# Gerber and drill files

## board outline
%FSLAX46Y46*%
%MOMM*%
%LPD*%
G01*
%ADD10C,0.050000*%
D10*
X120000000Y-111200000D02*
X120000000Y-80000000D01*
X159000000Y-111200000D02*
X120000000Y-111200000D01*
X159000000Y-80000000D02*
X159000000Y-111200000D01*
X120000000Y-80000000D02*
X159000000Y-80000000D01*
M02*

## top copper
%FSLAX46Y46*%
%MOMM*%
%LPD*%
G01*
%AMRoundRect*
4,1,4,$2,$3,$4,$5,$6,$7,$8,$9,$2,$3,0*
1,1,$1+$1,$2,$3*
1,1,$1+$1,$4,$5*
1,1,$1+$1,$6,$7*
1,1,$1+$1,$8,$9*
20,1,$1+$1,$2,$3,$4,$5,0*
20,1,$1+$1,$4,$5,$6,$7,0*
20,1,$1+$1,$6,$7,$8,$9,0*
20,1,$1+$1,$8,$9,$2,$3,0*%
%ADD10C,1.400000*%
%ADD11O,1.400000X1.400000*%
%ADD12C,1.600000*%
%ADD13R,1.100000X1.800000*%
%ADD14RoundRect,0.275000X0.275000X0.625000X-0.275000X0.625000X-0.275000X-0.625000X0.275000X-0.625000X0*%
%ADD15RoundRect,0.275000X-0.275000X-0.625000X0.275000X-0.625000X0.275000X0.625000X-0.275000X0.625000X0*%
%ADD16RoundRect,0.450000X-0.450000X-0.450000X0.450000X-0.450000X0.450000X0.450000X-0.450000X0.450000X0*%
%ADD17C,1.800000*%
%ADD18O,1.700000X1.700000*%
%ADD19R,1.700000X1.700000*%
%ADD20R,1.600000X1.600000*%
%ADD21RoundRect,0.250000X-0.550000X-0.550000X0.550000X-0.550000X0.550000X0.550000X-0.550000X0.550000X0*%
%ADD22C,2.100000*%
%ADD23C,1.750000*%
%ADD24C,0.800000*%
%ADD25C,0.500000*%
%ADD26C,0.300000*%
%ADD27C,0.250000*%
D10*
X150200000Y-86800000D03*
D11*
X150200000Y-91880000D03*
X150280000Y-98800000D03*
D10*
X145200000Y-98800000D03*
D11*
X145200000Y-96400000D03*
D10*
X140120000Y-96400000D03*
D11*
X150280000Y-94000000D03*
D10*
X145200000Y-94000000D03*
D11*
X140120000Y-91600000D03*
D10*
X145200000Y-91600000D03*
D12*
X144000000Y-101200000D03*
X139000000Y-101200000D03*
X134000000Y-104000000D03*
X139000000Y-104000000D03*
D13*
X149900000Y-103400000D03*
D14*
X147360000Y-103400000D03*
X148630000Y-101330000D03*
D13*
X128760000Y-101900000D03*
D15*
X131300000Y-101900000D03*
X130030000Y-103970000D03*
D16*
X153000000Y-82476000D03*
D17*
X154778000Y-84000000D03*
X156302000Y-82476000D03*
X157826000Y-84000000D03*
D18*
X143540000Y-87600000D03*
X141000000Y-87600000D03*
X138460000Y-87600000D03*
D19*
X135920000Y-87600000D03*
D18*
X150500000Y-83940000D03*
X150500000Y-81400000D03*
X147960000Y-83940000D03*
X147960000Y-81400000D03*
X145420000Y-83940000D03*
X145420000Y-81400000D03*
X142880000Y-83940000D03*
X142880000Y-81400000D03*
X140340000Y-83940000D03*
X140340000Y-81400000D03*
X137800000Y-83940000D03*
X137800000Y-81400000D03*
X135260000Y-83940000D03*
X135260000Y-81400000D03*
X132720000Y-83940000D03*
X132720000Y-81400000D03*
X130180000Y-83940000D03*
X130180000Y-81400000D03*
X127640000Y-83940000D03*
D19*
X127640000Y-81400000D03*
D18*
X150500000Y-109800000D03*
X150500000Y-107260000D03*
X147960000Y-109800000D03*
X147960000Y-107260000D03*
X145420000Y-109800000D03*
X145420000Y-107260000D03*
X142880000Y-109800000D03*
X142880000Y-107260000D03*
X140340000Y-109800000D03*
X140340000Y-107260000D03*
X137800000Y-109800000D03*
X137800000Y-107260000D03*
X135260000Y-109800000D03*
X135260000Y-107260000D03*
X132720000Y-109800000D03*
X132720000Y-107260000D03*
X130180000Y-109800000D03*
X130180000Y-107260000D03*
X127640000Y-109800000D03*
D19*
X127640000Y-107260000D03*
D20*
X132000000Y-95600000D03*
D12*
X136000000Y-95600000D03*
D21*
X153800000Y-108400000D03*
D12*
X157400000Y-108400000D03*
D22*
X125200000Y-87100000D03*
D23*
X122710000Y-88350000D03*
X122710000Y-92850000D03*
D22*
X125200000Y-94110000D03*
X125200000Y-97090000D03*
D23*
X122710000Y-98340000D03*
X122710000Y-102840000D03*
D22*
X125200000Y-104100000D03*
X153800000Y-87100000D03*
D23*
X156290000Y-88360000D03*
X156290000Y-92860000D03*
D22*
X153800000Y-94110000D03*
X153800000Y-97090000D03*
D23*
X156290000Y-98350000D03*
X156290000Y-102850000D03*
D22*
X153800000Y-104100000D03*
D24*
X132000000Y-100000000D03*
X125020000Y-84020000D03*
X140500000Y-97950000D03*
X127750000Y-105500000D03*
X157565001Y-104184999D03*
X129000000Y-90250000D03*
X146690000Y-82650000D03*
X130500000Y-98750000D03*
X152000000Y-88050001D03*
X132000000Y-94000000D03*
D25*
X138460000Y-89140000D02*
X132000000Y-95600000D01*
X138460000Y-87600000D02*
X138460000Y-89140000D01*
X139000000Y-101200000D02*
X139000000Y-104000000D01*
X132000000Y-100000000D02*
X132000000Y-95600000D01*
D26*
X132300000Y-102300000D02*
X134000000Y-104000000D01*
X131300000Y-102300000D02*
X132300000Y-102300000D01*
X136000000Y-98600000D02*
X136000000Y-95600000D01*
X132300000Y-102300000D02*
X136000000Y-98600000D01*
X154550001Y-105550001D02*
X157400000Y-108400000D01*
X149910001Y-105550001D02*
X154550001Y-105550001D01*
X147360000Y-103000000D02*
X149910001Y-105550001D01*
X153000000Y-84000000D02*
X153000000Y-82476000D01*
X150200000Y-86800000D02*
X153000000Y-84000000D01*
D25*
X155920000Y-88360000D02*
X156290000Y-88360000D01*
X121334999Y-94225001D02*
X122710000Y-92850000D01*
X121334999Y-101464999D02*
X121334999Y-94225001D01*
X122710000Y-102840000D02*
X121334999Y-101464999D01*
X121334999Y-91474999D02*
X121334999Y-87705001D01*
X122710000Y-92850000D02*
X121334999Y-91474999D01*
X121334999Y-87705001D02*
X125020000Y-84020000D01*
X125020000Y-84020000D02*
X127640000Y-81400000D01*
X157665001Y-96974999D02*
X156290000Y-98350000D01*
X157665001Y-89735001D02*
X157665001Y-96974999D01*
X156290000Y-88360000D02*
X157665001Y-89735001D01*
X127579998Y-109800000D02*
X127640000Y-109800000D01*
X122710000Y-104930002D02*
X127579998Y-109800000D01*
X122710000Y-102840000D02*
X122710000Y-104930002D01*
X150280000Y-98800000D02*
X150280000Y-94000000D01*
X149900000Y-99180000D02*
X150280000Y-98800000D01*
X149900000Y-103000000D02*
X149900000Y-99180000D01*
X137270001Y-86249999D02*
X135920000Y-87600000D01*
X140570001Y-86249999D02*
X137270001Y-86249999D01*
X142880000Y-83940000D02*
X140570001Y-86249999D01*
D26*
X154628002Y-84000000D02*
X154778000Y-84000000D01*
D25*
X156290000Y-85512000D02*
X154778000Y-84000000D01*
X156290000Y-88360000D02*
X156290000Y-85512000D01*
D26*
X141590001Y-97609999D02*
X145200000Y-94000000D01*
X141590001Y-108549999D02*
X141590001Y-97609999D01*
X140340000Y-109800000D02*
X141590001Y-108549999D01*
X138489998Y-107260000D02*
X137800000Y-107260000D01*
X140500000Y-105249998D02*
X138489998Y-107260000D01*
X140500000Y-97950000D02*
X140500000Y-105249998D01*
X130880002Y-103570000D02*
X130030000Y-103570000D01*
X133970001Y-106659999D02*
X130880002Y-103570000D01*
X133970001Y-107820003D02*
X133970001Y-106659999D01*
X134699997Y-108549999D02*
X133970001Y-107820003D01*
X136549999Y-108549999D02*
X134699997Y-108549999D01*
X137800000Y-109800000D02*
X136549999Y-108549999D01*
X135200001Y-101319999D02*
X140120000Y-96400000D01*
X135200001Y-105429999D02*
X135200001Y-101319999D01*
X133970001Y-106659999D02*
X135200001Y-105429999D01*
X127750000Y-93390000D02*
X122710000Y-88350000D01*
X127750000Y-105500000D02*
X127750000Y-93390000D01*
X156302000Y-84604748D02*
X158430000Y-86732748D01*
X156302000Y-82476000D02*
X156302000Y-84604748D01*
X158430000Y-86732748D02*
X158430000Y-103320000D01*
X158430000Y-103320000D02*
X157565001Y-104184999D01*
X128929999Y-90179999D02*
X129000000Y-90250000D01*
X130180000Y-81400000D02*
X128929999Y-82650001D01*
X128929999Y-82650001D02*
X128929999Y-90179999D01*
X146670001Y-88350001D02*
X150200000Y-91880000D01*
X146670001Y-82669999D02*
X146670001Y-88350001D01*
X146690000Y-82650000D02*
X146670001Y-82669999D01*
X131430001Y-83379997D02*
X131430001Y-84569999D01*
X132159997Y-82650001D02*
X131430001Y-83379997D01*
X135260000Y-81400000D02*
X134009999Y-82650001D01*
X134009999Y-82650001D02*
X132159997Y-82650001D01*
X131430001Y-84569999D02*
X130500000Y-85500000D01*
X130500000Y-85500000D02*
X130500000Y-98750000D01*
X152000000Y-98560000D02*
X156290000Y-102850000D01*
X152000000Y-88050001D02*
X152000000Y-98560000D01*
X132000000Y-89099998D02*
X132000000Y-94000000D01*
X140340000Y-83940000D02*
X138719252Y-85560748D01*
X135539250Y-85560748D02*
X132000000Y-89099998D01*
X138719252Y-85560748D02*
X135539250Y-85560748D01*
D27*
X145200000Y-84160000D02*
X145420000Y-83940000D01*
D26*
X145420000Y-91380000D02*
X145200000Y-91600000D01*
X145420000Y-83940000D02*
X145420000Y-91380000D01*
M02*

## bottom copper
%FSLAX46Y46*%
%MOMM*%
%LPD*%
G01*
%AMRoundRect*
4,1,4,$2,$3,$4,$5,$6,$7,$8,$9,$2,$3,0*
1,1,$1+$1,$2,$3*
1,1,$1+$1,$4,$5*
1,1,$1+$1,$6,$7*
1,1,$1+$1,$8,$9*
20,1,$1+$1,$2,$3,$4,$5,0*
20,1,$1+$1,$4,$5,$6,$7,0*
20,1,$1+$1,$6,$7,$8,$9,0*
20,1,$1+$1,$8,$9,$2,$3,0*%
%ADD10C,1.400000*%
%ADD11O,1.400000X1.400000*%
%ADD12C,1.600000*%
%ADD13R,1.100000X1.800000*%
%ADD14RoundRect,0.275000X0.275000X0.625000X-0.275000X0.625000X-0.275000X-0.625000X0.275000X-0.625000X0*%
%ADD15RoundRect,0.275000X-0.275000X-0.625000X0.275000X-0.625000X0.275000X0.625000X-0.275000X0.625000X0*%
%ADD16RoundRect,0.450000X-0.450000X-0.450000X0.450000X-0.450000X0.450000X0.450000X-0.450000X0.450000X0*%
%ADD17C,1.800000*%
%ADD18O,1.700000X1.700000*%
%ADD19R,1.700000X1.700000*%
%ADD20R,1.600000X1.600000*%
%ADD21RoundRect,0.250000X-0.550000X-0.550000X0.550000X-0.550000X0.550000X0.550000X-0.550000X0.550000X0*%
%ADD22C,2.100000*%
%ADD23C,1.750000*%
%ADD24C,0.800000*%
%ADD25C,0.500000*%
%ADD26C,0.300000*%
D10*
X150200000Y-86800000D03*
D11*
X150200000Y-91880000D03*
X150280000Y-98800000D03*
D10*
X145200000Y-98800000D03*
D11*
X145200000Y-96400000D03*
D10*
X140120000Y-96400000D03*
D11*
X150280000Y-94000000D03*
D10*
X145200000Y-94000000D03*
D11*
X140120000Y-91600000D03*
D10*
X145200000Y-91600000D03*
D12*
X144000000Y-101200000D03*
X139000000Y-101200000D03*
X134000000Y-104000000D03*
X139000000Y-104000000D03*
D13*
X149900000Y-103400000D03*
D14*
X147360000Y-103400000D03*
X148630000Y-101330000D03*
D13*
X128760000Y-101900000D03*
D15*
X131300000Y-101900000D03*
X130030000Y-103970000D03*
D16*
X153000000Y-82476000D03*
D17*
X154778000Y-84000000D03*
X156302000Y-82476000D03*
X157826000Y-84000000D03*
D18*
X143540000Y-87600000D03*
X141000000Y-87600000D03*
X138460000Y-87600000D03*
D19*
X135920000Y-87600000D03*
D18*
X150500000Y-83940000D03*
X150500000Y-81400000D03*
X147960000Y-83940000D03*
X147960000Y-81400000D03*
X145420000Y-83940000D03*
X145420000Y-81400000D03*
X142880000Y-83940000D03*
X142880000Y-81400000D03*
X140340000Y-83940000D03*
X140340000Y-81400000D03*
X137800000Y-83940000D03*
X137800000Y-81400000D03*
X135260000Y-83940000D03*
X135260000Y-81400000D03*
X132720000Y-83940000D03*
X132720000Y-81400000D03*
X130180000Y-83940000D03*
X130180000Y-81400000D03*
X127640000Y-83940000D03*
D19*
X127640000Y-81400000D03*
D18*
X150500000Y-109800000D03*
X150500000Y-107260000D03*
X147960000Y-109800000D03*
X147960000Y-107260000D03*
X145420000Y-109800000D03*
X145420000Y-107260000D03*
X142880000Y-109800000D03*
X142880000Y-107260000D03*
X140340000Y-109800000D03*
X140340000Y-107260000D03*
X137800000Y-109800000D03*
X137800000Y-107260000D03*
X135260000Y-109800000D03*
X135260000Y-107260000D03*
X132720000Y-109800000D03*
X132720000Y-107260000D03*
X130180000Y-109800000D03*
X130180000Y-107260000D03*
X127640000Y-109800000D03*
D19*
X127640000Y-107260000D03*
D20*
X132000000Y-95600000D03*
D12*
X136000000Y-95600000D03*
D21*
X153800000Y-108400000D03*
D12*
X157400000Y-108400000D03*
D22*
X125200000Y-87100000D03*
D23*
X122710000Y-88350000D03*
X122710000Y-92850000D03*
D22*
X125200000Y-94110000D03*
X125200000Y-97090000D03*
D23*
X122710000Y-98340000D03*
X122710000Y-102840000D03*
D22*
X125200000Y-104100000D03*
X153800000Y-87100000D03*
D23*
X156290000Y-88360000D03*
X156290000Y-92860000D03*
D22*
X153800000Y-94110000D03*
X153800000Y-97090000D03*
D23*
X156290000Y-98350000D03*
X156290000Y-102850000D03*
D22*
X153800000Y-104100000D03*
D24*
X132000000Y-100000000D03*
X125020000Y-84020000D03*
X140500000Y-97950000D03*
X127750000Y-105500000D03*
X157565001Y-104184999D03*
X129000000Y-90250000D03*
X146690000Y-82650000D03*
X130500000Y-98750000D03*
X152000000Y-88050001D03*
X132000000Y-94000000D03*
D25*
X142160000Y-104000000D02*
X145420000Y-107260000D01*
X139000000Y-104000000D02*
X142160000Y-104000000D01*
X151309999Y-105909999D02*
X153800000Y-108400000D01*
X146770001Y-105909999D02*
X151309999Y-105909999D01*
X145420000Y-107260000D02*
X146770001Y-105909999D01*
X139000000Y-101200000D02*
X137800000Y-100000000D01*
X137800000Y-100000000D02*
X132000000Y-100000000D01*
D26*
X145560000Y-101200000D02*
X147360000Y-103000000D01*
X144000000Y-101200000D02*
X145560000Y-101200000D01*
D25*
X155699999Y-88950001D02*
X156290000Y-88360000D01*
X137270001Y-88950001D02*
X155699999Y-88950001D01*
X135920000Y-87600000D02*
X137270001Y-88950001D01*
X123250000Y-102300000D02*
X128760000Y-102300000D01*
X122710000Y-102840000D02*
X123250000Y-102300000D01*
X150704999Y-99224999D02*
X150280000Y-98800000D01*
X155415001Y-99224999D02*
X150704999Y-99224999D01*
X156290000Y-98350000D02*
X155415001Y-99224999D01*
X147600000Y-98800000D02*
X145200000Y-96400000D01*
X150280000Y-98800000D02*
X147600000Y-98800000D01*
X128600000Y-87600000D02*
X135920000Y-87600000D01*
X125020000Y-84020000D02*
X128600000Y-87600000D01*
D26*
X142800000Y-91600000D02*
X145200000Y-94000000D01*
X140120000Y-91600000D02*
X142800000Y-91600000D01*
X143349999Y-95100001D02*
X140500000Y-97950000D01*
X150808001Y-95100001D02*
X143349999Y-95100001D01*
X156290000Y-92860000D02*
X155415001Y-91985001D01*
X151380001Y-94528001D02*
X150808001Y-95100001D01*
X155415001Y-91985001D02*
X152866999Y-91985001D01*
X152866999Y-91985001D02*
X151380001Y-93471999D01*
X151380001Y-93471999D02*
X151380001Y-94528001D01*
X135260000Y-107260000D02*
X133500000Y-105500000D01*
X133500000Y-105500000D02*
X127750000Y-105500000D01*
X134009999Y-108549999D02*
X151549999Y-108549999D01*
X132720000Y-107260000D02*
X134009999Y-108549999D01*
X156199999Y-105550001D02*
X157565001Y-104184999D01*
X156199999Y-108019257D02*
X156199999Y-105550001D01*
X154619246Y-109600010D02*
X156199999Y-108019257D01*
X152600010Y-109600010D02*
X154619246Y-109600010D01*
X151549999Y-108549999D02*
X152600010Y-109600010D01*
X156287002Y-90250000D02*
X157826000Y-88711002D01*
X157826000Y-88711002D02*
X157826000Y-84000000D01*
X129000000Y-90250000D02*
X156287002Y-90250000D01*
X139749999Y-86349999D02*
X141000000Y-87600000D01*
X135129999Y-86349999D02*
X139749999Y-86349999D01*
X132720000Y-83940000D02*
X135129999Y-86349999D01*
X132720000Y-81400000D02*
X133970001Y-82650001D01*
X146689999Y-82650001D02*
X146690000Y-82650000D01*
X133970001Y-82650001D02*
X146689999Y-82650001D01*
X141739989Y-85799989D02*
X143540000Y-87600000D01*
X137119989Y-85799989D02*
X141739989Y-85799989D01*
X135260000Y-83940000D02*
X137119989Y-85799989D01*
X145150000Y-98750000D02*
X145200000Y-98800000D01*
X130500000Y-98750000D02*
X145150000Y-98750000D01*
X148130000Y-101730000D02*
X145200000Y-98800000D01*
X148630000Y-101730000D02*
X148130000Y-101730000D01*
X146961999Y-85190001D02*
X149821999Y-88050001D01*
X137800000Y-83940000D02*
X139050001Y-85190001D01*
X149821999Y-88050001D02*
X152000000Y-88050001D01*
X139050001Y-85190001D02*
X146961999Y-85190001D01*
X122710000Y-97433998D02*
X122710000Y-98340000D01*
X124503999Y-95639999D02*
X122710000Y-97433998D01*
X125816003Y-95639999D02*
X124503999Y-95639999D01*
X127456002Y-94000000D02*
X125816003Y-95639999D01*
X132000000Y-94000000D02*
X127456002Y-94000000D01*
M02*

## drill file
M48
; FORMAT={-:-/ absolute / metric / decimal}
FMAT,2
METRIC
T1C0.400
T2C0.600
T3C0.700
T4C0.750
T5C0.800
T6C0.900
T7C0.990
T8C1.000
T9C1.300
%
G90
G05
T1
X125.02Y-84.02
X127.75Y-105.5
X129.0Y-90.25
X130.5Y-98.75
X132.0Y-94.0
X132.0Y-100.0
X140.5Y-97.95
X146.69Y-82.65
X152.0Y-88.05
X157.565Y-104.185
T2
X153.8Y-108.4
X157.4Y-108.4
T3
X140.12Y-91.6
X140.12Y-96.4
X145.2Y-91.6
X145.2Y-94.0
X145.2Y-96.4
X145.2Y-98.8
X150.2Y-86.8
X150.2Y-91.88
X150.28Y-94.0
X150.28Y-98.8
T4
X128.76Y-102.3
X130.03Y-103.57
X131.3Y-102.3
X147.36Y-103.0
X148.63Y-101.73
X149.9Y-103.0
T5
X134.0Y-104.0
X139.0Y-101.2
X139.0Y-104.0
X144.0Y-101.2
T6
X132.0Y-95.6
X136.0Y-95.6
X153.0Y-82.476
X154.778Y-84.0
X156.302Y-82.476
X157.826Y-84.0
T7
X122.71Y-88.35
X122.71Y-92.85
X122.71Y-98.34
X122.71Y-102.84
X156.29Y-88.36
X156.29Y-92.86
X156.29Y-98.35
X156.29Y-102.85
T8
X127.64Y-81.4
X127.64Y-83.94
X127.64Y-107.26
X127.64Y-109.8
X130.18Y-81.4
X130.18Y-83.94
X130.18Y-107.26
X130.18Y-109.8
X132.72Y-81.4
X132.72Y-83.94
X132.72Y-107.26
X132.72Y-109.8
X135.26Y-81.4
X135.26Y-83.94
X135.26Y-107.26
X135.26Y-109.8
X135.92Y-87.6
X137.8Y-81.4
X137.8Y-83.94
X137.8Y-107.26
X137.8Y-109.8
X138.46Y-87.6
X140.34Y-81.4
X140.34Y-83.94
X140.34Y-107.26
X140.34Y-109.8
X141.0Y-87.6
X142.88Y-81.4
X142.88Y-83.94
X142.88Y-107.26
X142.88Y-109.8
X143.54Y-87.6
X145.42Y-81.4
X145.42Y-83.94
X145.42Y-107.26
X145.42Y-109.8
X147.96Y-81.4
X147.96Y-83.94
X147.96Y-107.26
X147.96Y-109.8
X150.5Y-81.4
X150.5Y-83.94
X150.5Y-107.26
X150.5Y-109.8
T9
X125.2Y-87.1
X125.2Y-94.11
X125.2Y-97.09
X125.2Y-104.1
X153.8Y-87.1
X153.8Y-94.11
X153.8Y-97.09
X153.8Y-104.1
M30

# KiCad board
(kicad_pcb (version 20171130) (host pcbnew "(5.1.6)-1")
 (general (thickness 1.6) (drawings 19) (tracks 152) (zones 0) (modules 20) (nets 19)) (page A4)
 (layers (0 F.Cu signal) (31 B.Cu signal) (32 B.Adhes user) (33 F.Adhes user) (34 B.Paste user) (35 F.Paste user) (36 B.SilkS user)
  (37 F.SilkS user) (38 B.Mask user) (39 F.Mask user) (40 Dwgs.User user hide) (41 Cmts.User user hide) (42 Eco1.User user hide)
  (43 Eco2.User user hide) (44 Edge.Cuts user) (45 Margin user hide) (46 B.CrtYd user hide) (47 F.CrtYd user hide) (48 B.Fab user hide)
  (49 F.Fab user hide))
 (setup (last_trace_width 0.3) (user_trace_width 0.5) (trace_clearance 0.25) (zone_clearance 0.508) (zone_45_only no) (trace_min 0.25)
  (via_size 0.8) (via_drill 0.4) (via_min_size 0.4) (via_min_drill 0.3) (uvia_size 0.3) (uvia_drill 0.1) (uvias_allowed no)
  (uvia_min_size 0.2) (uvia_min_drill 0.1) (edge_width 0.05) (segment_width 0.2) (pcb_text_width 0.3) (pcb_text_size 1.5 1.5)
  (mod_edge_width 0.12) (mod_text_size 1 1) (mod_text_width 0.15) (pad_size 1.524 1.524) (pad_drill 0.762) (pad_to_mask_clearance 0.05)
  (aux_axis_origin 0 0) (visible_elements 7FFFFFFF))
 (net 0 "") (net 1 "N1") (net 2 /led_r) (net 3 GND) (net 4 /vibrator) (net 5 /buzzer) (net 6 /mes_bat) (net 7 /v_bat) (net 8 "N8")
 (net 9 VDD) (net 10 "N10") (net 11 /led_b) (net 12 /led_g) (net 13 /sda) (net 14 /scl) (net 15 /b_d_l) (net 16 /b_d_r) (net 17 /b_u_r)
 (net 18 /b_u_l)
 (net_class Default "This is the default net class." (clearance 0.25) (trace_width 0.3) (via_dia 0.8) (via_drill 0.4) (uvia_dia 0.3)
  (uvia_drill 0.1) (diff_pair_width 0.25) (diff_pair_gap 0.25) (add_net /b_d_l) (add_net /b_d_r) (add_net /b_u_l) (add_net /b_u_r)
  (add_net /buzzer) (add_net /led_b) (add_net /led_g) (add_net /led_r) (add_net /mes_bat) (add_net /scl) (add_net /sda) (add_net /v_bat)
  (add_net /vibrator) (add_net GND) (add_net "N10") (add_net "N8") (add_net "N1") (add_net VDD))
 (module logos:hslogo (layer F.Cu) (at 122.7 108)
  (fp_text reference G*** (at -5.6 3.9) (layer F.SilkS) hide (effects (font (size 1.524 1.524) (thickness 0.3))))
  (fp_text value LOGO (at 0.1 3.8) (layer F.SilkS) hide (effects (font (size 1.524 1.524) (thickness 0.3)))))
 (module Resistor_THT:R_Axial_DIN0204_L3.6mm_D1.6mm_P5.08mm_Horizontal (layer B.Cu) (at 150.2 86.8 270)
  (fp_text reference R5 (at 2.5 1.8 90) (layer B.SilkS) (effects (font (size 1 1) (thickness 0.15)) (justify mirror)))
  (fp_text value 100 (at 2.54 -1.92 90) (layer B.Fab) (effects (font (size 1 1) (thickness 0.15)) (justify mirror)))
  (pad 1 thru_hole circle (at 0 0 270) (size 1.4 1.4) (drill 0.7) (layers *.Cu *.Mask) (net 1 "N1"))
  (pad 2 thru_hole oval (at 5.08 0 270) (size 1.4 1.4) (drill 0.7) (layers *.Cu *.Mask) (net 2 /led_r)))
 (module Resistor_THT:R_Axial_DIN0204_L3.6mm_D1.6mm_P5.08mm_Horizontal (layer B.Cu) (at 145.2 98.8)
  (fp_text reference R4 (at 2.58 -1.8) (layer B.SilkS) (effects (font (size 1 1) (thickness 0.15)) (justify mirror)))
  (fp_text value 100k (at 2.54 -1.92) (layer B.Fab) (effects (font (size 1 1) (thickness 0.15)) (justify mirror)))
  (pad 2 thru_hole oval (at 5.08 0) (size 1.4 1.4) (drill 0.7) (layers *.Cu *.Mask) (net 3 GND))
  (pad 1 thru_hole circle (at 0 0) (size 1.4 1.4) (drill 0.7) (layers *.Cu *.Mask) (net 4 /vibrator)))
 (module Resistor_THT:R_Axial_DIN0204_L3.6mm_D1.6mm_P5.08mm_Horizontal (layer B.Cu) (at 140.12 96.4)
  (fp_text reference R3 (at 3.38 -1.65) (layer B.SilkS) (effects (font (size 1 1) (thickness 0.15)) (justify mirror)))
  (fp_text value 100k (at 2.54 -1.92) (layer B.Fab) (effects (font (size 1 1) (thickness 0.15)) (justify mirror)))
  (pad 2 thru_hole oval (at 5.08 0) (size 1.4 1.4) (drill 0.7) (layers *.Cu *.Mask) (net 3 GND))
  (pad 1 thru_hole circle (at 0 0) (size 1.4 1.4) (drill 0.7) (layers *.Cu *.Mask) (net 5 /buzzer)))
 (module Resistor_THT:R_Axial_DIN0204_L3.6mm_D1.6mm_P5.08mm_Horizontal (layer B.Cu) (at 145.2 94)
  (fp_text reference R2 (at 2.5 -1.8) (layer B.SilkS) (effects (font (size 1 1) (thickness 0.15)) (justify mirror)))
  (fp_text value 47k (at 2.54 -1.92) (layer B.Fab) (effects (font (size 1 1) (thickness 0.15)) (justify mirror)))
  (pad 2 thru_hole oval (at 5.08 0) (size 1.4 1.4) (drill 0.7) (layers *.Cu *.Mask) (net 3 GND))
  (pad 1 thru_hole circle (at 0 0) (size 1.4 1.4) (drill 0.7) (layers *.Cu *.Mask) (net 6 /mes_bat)))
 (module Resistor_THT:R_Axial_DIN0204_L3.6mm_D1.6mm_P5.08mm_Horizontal (layer B.Cu) (at 145.2 91.6 180)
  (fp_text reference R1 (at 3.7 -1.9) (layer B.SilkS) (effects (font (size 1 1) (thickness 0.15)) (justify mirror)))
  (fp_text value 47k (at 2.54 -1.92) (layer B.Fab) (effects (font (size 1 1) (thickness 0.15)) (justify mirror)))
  (pad 2 thru_hole oval (at 5.08 0 180) (size 1.4 1.4) (drill 0.7) (layers *.Cu *.Mask) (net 6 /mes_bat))
  (pad 1 thru_hole circle (at 0 0 180) (size 1.4 1.4) (drill 0.7) (layers *.Cu *.Mask) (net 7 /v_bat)))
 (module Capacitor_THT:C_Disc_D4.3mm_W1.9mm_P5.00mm (layer B.Cu) (at 139 101.2)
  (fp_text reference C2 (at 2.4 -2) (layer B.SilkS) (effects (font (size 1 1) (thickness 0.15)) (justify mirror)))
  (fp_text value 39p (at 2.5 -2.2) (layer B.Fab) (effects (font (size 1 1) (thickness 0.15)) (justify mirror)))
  (pad 2 thru_hole circle (at 5 0) (size 1.6 1.6) (drill 0.8) (layers *.Cu *.Mask) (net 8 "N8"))
  (pad 1 thru_hole circle (at 0 0) (size 1.6 1.6) (drill 0.8) (layers *.Cu *.Mask) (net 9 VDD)))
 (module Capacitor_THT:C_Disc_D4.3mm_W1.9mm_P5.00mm (layer B.Cu) (at 139 104 180)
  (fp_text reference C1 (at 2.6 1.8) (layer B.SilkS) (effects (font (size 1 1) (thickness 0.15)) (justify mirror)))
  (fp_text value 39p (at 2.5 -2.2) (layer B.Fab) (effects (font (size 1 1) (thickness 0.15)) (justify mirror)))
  (pad 2 thru_hole circle (at 5 0 180) (size 1.6 1.6) (drill 0.8) (layers *.Cu *.Mask) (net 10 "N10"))
  (pad 1 thru_hole circle (at 0 0 180) (size 1.6 1.6) (drill 0.8) (layers *.Cu *.Mask) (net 9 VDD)))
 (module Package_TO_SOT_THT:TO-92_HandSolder (layer B.Cu) (at 149.9 103 180)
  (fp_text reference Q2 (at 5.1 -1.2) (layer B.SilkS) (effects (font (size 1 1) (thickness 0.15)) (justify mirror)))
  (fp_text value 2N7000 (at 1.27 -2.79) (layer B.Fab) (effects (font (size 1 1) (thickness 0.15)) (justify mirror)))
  (pad 1 thru_hole rect (at 0 0 180) (size 1.1 1.8) (drill 0.75 (offset 0 -0.4)) (layers *.Cu *.Mask) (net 3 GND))
  (pad 3 thru_hole roundrect (at 2.54 0 180) (size 1.1 1.8) (drill 0.75 (offset 0 -0.4)) (layers *.Cu *.Mask) (roundrect_rratio 0.25)
   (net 8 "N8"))
  (pad 2 thru_hole roundrect (at 1.27 1.27 180) (size 1.1 1.8) (drill 0.75 (offset 0 0.4)) (layers *.Cu *.Mask) (roundrect_rratio 0.25)
   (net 4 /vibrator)))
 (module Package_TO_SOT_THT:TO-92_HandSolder (layer B.Cu) (at 128.76 102.3)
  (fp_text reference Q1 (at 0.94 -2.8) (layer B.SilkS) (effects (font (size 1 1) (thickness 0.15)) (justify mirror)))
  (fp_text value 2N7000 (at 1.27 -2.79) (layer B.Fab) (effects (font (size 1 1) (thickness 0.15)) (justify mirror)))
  (pad 1 thru_hole rect (at 0 0) (size 1.1 1.8) (drill 0.75 (offset 0 -0.4)) (layers *.Cu *.Mask) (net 3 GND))
  (pad 3 thru_hole roundrect (at 2.54 0) (size 1.1 1.8) (drill 0.75 (offset 0 -0.4)) (layers *.Cu *.Mask) (roundrect_rratio 0.25)
   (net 10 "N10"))
  (pad 2 thru_hole roundrect (at 1.27 1.27) (size 1.1 1.8) (drill 0.75 (offset 0 0.4)) (layers *.Cu *.Mask) (roundrect_rratio 0.25)
   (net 5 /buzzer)))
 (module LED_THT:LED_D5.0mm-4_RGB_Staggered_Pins (layer F.Cu) (at 153 82.476)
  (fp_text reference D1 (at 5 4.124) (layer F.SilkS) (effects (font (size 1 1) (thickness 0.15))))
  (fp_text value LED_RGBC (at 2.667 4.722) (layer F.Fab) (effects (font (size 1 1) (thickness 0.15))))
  (pad 1 thru_hole roundrect (at 0 0) (size 1.8 1.8) (drill 0.9) (layers *.Cu *.Mask) (roundrect_rratio 0.25) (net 1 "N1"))
  (pad 2 thru_hole circle (at 1.778 1.524) (size 1.8 1.8) (drill 0.9) (layers *.Cu *.Mask) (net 3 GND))
  (pad 3 thru_hole circle (at 3.302 0) (size 1.8 1.8) (drill 0.9) (layers *.Cu *.Mask) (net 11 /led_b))
  (pad 4 thru_hole circle (at 4.826 1.524) (size 1.8 1.8) (drill 0.9) (layers *.Cu *.Mask) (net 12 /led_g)))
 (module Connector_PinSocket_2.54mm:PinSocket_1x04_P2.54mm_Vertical (layer F.Cu) (at 135.92 87.6 90)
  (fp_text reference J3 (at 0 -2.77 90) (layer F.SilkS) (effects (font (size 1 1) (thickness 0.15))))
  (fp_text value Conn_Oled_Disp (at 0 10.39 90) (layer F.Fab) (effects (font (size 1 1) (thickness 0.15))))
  (pad 4 thru_hole oval (at 0 7.62 90) (size 1.7 1.7) (drill 1) (layers *.Cu *.Mask) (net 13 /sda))
  (pad 3 thru_hole oval (at 0 5.08 90) (size 1.7 1.7) (drill 1) (layers *.Cu *.Mask) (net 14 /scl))
  (pad 2 thru_hole oval (at 0 2.54 90) (size 1.7 1.7) (drill 1) (layers *.Cu *.Mask) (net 9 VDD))
  (pad 1 thru_hole rect (at 0 0 90) (size 1.7 1.7) (drill 1) (layers *.Cu *.Mask) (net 3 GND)))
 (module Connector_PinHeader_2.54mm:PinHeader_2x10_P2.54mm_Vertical (layer B.Cu) (at 127.64 81.4 270)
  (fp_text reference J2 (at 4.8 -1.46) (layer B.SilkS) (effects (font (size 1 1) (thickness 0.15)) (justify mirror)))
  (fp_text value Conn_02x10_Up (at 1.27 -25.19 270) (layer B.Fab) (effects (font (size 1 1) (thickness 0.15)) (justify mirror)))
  (pad 20 thru_hole oval (at 2.54 -22.86 270) (size 1.7 1.7) (drill 1) (layers *.Cu *.Mask))
  (pad 19 thru_hole oval (at 0 -22.86 270) (size 1.7 1.7) (drill 1) (layers *.Cu *.Mask))
  (pad 18 thru_hole oval (at 2.54 -20.32 270) (size 1.7 1.7) (drill 1) (layers *.Cu *.Mask))
  (pad 17 thru_hole oval (at 0 -20.32 270) (size 1.7 1.7) (drill 1) (layers *.Cu *.Mask))
  (pad 16 thru_hole oval (at 2.54 -17.78 270) (size 1.7 1.7) (drill 1) (layers *.Cu *.Mask) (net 7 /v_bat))
  (pad 15 thru_hole oval (at 0 -17.78 270) (size 1.7 1.7) (drill 1) (layers *.Cu *.Mask))
  (pad 14 thru_hole oval (at 2.54 -15.24 270) (size 1.7 1.7) (drill 1) (layers *.Cu *.Mask) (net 3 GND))
  (pad 13 thru_hole oval (at 0 -15.24 270) (size 1.7 1.7) (drill 1) (layers *.Cu *.Mask))
  (pad 12 thru_hole oval (at 2.54 -12.7 270) (size 1.7 1.7) (drill 1) (layers *.Cu *.Mask) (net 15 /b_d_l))
  (pad 11 thru_hole oval (at 0 -12.7 270) (size 1.7 1.7) (drill 1) (layers *.Cu *.Mask))
  (pad 10 thru_hole oval (at 2.54 -10.16 270) (size 1.7 1.7) (drill 1) (layers *.Cu *.Mask) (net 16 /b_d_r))
  (pad 9 thru_hole oval (at 0 -10.16 270) (size 1.7 1.7) (drill 1) (layers *.Cu *.Mask))
  (pad 8 thru_hole oval (at 2.54 -7.62 270) (size 1.7 1.7) (drill 1) (layers *.Cu *.Mask) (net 13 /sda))
  (pad 7 thru_hole oval (at 0 -7.62 270) (size 1.7 1.7) (drill 1) (layers *.Cu *.Mask) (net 4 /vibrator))
  (pad 6 thru_hole oval (at 2.54 -5.08 270) (size 1.7 1.7) (drill 1) (layers *.Cu *.Mask) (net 14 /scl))
  (pad 5 thru_hole oval (at 0 -5.08 270) (size 1.7 1.7) (drill 1) (layers *.Cu *.Mask) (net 2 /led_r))
  (pad 4 thru_hole oval (at 2.54 -2.54 270) (size 1.7 1.7) (drill 1) (layers *.Cu *.Mask))
  (pad 3 thru_hole oval (at 0 -2.54 270) (size 1.7 1.7) (drill 1) (layers *.Cu *.Mask) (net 12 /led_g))
  (pad 2 thru_hole oval (at 2.54 0 270) (size 1.7 1.7) (drill 1) (layers *.Cu *.Mask))
  (pad 1 thru_hole rect (at 0 0 270) (size 1.7 1.7) (drill 1) (layers *.Cu *.Mask) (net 3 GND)))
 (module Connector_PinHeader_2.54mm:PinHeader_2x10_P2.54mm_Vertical (layer B.Cu) (at 127.64 107.26 270)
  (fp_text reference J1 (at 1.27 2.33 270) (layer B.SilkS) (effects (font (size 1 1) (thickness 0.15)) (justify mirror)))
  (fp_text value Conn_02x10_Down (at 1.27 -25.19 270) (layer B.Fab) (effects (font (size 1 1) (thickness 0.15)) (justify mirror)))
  (pad 20 thru_hole oval (at 2.54 -22.86 270) (size 1.7 1.7) (drill 1) (layers *.Cu *.Mask))
  (pad 19 thru_hole oval (at 0 -22.86 270) (size 1.7 1.7) (drill 1) (layers *.Cu *.Mask))
  (pad 18 thru_hole oval (at 2.54 -20.32 270) (size 1.7 1.7) (drill 1) (layers *.Cu *.Mask))
  (pad 17 thru_hole oval (at 0 -20.32 270) (size 1.7 1.7) (drill 1) (layers *.Cu *.Mask))
  (pad 16 thru_hole oval (at 2.54 -17.78 270) (size 1.7 1.7) (drill 1) (layers *.Cu *.Mask))
  (pad 15 thru_hole oval (at 0 -17.78 270) (size 1.7 1.7) (drill 1) (layers *.Cu *.Mask) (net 9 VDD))
  (pad 14 thru_hole oval (at 2.54 -15.24 270) (size 1.7 1.7) (drill 1) (layers *.Cu *.Mask))
  (pad 13 thru_hole oval (at 0 -15.24 270) (size 1.7 1.7) (drill 1) (layers *.Cu *.Mask))
  (pad 12 thru_hole oval (at 2.54 -12.7 270) (size 1.7 1.7) (drill 1) (layers *.Cu *.Mask) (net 6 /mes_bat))
  (pad 11 thru_hole oval (at 0 -12.7 270) (size 1.7 1.7) (drill 1) (layers *.Cu *.Mask))
  (pad 10 thru_hole oval (at 2.54 -10.16 270) (size 1.7 1.7) (drill 1) (layers *.Cu *.Mask) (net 5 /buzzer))
  (pad 9 thru_hole oval (at 0 -10.16 270) (size 1.7 1.7) (drill 1) (layers *.Cu *.Mask) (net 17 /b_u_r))
  (pad 8 thru_hole oval (at 2.54 -7.62 270) (size 1.7 1.7) (drill 1) (layers *.Cu *.Mask))
  (pad 7 thru_hole oval (at 0 -7.62 270) (size 1.7 1.7) (drill 1) (layers *.Cu *.Mask) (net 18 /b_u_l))
  (pad 6 thru_hole oval (at 2.54 -5.08 270) (size 1.7 1.7) (drill 1) (layers *.Cu *.Mask))
  (pad 5 thru_hole oval (at 0 -5.08 270) (size 1.7 1.7) (drill 1) (layers *.Cu *.Mask) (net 11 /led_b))
  (pad 4 thru_hole oval (at 2.54 -2.54 270) (size 1.7 1.7) (drill 1) (layers *.Cu *.Mask))
  (pad 3 thru_hole oval (at 0 -2.54 270) (size 1.7 1.7) (drill 1) (layers *.Cu *.Mask))
  (pad 2 thru_hole oval (at 2.54 0 270) (size 1.7 1.7) (drill 1) (layers *.Cu *.Mask) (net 3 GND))
  (pad 1 thru_hole rect (at 0 0 270) (size 1.7 1.7) (drill 1) (layers *.Cu *.Mask)))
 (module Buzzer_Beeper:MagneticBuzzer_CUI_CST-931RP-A (layer B.Cu) (at 132 95.6 270)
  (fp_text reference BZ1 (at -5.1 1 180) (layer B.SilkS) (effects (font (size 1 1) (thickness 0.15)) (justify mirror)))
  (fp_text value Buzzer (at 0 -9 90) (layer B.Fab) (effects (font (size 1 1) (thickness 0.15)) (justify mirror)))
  (pad 1 thru_hole rect (at 0 0 270) (size 1.6 1.6) (drill 0.9) (layers *.Cu *.Mask) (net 9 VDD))
  (pad 2 thru_hole circle (at 0 -4 270) (size 1.6 1.6) (drill 0.9) (layers *.Cu *.Mask) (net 10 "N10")))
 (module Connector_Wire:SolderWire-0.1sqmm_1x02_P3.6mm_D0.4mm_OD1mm (layer F.Cu) (at 153.8 108.4)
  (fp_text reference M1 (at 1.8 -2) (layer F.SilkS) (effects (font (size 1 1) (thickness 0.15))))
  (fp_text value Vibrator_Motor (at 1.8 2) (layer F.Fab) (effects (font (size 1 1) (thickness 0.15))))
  (pad 1 thru_hole roundrect (at 0 0) (size 1.6 1.6) (drill 0.6) (layers *.Cu *.Mask) (roundrect_rratio 0.15625) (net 9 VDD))
  (pad 2 thru_hole circle (at 3.6 0) (size 1.6 1.6) (drill 0.6) (layers *.Cu *.Mask) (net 8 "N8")))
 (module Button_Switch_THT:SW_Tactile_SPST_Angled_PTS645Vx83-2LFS (layer B.Cu) (at 122.71 88.35 270)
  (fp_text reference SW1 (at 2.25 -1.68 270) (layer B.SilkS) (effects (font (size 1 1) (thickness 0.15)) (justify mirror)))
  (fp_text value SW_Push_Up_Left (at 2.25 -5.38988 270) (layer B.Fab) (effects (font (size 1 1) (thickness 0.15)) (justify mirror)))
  (pad "" thru_hole circle (at -1.25 -2.49 270) (size 2.1 2.1) (drill 1.3) (layers *.Cu *.Mask))
  (pad 1 thru_hole circle (at 0 0 270) (size 1.75 1.75) (drill 0.99) (layers *.Cu *.Mask) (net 18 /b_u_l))
  (pad 2 thru_hole circle (at 4.5 0 270) (size 1.75 1.75) (drill 0.99) (layers *.Cu *.Mask) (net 3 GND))
  (pad "" thru_hole circle (at 5.76 -2.49 270) (size 2.1 2.1) (drill 1.3) (layers *.Cu *.Mask)))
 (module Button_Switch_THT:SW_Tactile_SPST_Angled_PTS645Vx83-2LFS (layer B.Cu) (at 122.71 98.34 270)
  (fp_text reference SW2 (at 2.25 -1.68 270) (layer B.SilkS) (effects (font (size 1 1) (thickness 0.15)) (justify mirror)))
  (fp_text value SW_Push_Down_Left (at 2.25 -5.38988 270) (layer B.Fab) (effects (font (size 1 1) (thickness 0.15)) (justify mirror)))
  (pad "" thru_hole circle (at -1.25 -2.49 270) (size 2.1 2.1) (drill 1.3) (layers *.Cu *.Mask))
  (pad 1 thru_hole circle (at 0 0 270) (size 1.75 1.75) (drill 0.99) (layers *.Cu *.Mask) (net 15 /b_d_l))
  (pad 2 thru_hole circle (at 4.5 0 270) (size 1.75 1.75) (drill 0.99) (layers *.Cu *.Mask) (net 3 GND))
  (pad "" thru_hole circle (at 5.76 -2.49 270) (size 2.1 2.1) (drill 1.3) (layers *.Cu *.Mask)))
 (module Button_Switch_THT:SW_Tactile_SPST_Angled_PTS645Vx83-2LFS (layer B.Cu) (at 156.29 92.86 90)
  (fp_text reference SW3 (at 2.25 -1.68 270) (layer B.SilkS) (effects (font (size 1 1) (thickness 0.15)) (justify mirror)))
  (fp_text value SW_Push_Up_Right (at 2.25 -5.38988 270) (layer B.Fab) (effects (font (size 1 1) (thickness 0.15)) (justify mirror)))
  (pad "" thru_hole circle (at 5.76 -2.49 90) (size 2.1 2.1) (drill 1.3) (layers *.Cu *.Mask))
  (pad 2 thru_hole circle (at 4.5 0 90) (size 1.75 1.75) (drill 0.99) (layers *.Cu *.Mask) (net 3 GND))
  (pad 1 thru_hole circle (at 0 0 90) (size 1.75 1.75) (drill 0.99) (layers *.Cu *.Mask) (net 17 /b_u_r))
  (pad "" thru_hole circle (at -1.25 -2.49 90) (size 2.1 2.1) (drill 1.3) (layers *.Cu *.Mask)))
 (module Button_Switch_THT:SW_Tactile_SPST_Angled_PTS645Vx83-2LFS (layer B.Cu) (at 156.29 102.85 90)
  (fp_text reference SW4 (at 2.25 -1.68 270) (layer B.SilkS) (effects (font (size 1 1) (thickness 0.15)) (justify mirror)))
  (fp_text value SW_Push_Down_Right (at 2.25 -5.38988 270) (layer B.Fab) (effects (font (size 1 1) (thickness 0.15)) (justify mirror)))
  (pad "" thru_hole circle (at 5.76 -2.49 90) (size 2.1 2.1) (drill 1.3) (layers *.Cu *.Mask))
  (pad 2 thru_hole circle (at 4.5 0 90) (size 1.75 1.75) (drill 0.99) (layers *.Cu *.Mask) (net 3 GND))
  (pad 1 thru_hole circle (at 0 0 90) (size 1.75 1.75) (drill 0.99) (layers *.Cu *.Mask) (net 16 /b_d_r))
  (pad "" thru_hole circle (at -1.25 -2.49 90) (size 2.1 2.1) (drill 1.3) (layers *.Cu *.Mask)))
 (gr_line (start 120 111.2) (end 120 80) (layer Edge.Cuts) (width 0.05))
 (gr_line (start 159 111.2) (end 120 111.2) (layer Edge.Cuts) (width 0.05))
 (gr_line (start 159 80) (end 159 111.2) (layer Edge.Cuts) (width 0.05))
 (gr_line (start 120 80) (end 159 80) (layer Edge.Cuts) (width 0.05))
 (segment (start 138.46 89.14) (end 132 95.6) (width 0.5) (layer F.Cu) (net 9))
 (segment (start 138.46 87.6) (end 138.46 89.14) (width 0.5) (layer F.Cu) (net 9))
 (segment (start 139 101.2) (end 139 104) (width 0.5) (layer F.Cu) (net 9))
 (segment (start 142.16 104) (end 145.42 107.26) (width 0.5) (layer B.Cu) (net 9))
 (segment (start 139 104) (end 142.16 104) (width 0.5) (layer B.Cu) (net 9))
 (segment (start 151.309999 105.909999) (end 153.8 108.4) (width 0.5) (layer B.Cu) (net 9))
 (segment (start 146.770001 105.909999) (end 151.309999 105.909999) (width 0.5) (layer B.Cu) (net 9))
 (segment (start 145.42 107.26) (end 146.770001 105.909999) (width 0.5) (layer B.Cu) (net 9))
 (segment (start 139 101.2) (end 137.8 100) (width 0.5) (layer B.Cu) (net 9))
 (via (at 132 100) (size 0.8) (drill 0.4) (layers F.Cu B.Cu) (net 9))
 (segment (start 137.8 100) (end 132 100) (width 0.5) (layer B.Cu) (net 9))
 (segment (start 132 100) (end 132 95.6) (width 0.5) (layer F.Cu) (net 9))
 (segment (start 132.3 102.3) (end 134 104) (width 0.3) (layer F.Cu) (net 10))
 (segment (start 131.3 102.3) (end 132.3 102.3) (width 0.3) (layer F.Cu) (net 10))
 (segment (start 136 98.6) (end 136 95.6) (width 0.3) (layer F.Cu) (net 10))
 (segment (start 132.3 102.3) (end 136 98.6) (width 0.3) (layer F.Cu) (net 10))
 (segment (start 145.56 101.2) (end 147.36 103) (width 0.3) (layer B.Cu) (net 8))
 (segment (start 144 101.2) (end 145.56 101.2) (width 0.3) (layer B.Cu) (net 8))
 (segment (start 154.550001 105.550001) (end 157.4 108.4) (width 0.3) (layer F.Cu) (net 8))
 (segment (start 149.910001 105.550001) (end 154.550001 105.550001) (width 0.3) (layer F.Cu) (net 8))
 (segment (start 147.36 103) (end 149.910001 105.550001) (width 0.3) (layer F.Cu) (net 8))
 (segment (start 153 84) (end 153 82.476) (width 0.3) (layer F.Cu) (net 1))
 (segment (start 150.2 86.8) (end 153 84) (width 0.3) (layer F.Cu) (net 1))
 (segment (start 155.92 88.36) (end 156.29 88.36) (width 0.5) (layer F.Cu) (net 3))
 (segment (start 121.334999 94.225001) (end 122.71 92.85) (width 0.5) (layer F.Cu) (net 3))
 (segment (start 121.334999 101.464999) (end 121.334999 94.225001) (width 0.5) (layer F.Cu) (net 3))
 (segment (start 122.71 102.84) (end 121.334999 101.464999) (width 0.5) (layer F.Cu) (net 3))
 (segment (start 121.334999 91.474999) (end 121.334999 87.705001) (width 0.5) (layer F.Cu) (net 3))
 (segment (start 122.71 92.85) (end 121.334999 91.474999) (width 0.5) (layer F.Cu) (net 3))
 (segment (start 121.334999 87.705001) (end 125.02 84.02) (width 0.5) (layer F.Cu) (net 3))
 (via (at 125.02 84.02) (size 0.8) (drill 0.4) (layers F.Cu B.Cu) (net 3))
 (segment (start 125.02 84.02) (end 127.64 81.4) (width 0.5) (layer F.Cu) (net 3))
 (segment (start 155.699999 88.950001) (end 156.29 88.36) (width 0.5) (layer B.Cu) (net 3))
 (segment (start 137.270001 88.950001) (end 155.699999 88.950001) (width 0.5) (layer B.Cu) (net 3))
 (segment (start 135.92 87.6) (end 137.270001 88.950001) (width 0.5) (layer B.Cu) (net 3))
 (segment (start 157.665001 96.974999) (end 156.29 98.35) (width 0.5) (layer F.Cu) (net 3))
 (segment (start 157.665001 89.735001) (end 157.665001 96.974999) (width 0.5) (layer F.Cu) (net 3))
 (segment (start 156.29 88.36) (end 157.665001 89.735001) (width 0.5) (layer F.Cu) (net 3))
 (segment (start 127.579998 109.8) (end 127.64 109.8) (width 0.5) (layer F.Cu) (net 3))
 (segment (start 122.71 104.930002) (end 127.579998 109.8) (width 0.5) (layer F.Cu) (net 3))
 (segment (start 122.71 102.84) (end 122.71 104.930002) (width 0.5) (layer F.Cu) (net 3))
 (segment (start 123.25 102.3) (end 128.76 102.3) (width 0.5) (layer B.Cu) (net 3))
 (segment (start 122.71 102.84) (end 123.25 102.3) (width 0.5) (layer B.Cu) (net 3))
 (segment (start 150.704999 99.224999) (end 150.28 98.8) (width 0.5) (layer B.Cu) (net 3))
 (segment (start 155.415001 99.224999) (end 150.704999 99.224999) (width 0.5) (layer B.Cu) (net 3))
 (segment (start 156.29 98.35) (end 155.415001 99.224999) (width 0.5) (layer B.Cu) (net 3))
 (segment (start 147.6 98.8) (end 145.2 96.4) (width 0.5) (layer B.Cu) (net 3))
 (segment (start 150.28 98.8) (end 147.6 98.8) (width 0.5) (layer B.Cu) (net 3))
 (segment (start 150.28 98.8) (end 150.28 94) (width 0.5) (layer F.Cu) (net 3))
 (segment (start 149.9 99.18) (end 150.28 98.8) (width 0.5) (layer F.Cu) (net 3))
 (segment (start 149.9 103) (end 149.9 99.18) (width 0.5) (layer F.Cu) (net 3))
 (segment (start 128.6 87.6) (end 135.92 87.6) (width 0.5) (layer B.Cu) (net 3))
 (segment (start 125.02 84.02) (end 128.6 87.6) (width 0.5) (layer B.Cu) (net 3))
 (segment (start 137.270001 86.249999) (end 135.92 87.6) (width 0.5) (layer F.Cu) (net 3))
 (segment (start 140.570001 86.249999) (end 137.270001 86.249999) (width 0.5) (layer F.Cu) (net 3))
 (segment (start 142.88 83.94) (end 140.570001 86.249999) (width 0.5) (layer F.Cu) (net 3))
 (segment (start 154.628002 84) (end 154.778 84) (width 0.3) (layer F.Cu) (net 3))
 (segment (start 156.29 85.512) (end 154.778 84) (width 0.5) (layer F.Cu) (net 3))
 (segment (start 156.29 88.36) (end 156.29 85.512) (width 0.5) (layer F.Cu) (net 3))
 (segment (start 141.590001 97.609999) (end 145.2 94) (width 0.3) (layer F.Cu) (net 6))
 (segment (start 141.590001 108.549999) (end 141.590001 97.609999) (width 0.3) (layer F.Cu) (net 6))
 (segment (start 140.34 109.8) (end 141.590001 108.549999) (width 0.3) (layer F.Cu) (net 6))
 (segment (start 142.8 91.6) (end 145.2 94) (width 0.3) (layer B.Cu) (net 6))
 (segment (start 140.12 91.6) (end 142.8 91.6) (width 0.3) (layer B.Cu) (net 6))
 (via (at 140.5 97.95) (size 0.8) (drill 0.4) (layers F.Cu B.Cu) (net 17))
 (segment (start 143.349999 95.100001) (end 140.5 97.95) (width 0.3) (layer B.Cu) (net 17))
 (segment (start 150.808001 95.100001) (end 143.349999 95.100001) (width 0.3) (layer B.Cu) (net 17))
 (segment (start 156.29 92.86) (end 155.415001 91.985001) (width 0.3) (layer B.Cu) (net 17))
 (segment (start 151.380001 94.528001) (end 150.808001 95.100001) (width 0.3) (layer B.Cu) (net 17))
 (segment (start 155.415001 91.985001) (end 152.866999 91.985001) (width 0.3) (layer B.Cu) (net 17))
 (segment (start 152.866999 91.985001) (end 151.380001 93.471999) (width 0.3) (layer B.Cu) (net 17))
 (segment (start 151.380001 93.471999) (end 151.380001 94.528001) (width 0.3) (layer B.Cu) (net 17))
 (segment (start 138.489998 107.26) (end 137.8 107.26) (width 0.3) (layer F.Cu) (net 17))
 (segment (start 140.5 105.249998) (end 138.489998 107.26) (width 0.3) (layer F.Cu) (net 17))
 (segment (start 140.5 97.95) (end 140.5 105.249998) (width 0.3) (layer F.Cu) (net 17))
 (segment (start 130.880002 103.57) (end 130.03 103.57) (width 0.3) (layer F.Cu) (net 5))
 (segment (start 133.970001 106.659999) (end 130.880002 103.57) (width 0.3) (layer F.Cu) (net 5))
 (segment (start 133.970001 107.820003) (end 133.970001 106.659999) (width 0.3) (layer F.Cu) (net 5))
 (segment (start 134.699997 108.549999) (end 133.970001 107.820003) (width 0.3) (layer F.Cu) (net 5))
 (segment (start 136.549999 108.549999) (end 134.699997 108.549999) (width 0.3) (layer F.Cu) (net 5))
 (segment (start 137.8 109.8) (end 136.549999 108.549999) (width 0.3) (layer F.Cu) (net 5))
 (segment (start 135.200001 101.319999) (end 140.12 96.4) (width 0.3) (layer F.Cu) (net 5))
 (segment (start 135.200001 105.429999) (end 135.200001 101.319999) (width 0.3) (layer F.Cu) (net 5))
 (segment (start 133.970001 106.659999) (end 135.200001 105.429999) (width 0.3) (layer F.Cu) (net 5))
 (via (at 127.75 105.5) (size 0.8) (drill 0.4) (layers F.Cu B.Cu) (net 18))
 (segment (start 135.26 107.26) (end 133.5 105.5) (width 0.3) (layer B.Cu) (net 18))
 (segment (start 133.5 105.5) (end 127.75 105.5) (width 0.3) (layer B.Cu) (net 18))
 (segment (start 127.75 93.39) (end 122.71 88.35) (width 0.3) (layer F.Cu) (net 18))
 (segment (start 127.75 105.5) (end 127.75 93.39) (width 0.3) (layer F.Cu) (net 18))
 (segment (start 134.009999 108.549999) (end 151.549999 108.549999) (width 0.3) (layer B.Cu) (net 11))
 (segment (start 132.72 107.26) (end 134.009999 108.549999) (width 0.3) (layer B.Cu) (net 11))
 (segment (start 156.199999 105.550001) (end 157.565001 104.184999) (width 0.3) (layer B.Cu) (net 11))
 (segment (start 156.199999 108.019257) (end 156.199999 105.550001) (width 0.3) (layer B.Cu) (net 11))
 (segment (start 154.619246 109.60001) (end 156.199999 108.019257) (width 0.3) (layer B.Cu) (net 11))
 (segment (start 152.60001 109.60001) (end 154.619246 109.60001) (width 0.3) (layer B.Cu) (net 11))
 (segment (start 151.549999 108.549999) (end 152.60001 109.60001) (width 0.3) (layer B.Cu) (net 11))
 (segment (start 156.302 84.604748) (end 158.43 86.732748) (width 0.3) (layer F.Cu) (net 11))
 (segment (start 156.302 82.476) (end 156.302 84.604748) (width 0.3) (layer F.Cu) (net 11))
 (via (at 157.565001 104.184999) (size 0.8) (drill 0.4) (layers F.Cu B.Cu) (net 11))
 (segment (start 158.43 86.732748) (end 158.43 103.32) (width 0.3) (layer F.Cu) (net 11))
 (segment (start 158.43 103.32) (end 157.565001 104.184999) (width 0.3) (layer F.Cu) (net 11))
 (via (at 129 90.25) (size 0.8) (drill 0.4) (layers F.Cu B.Cu) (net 12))
 (segment (start 128.929999 90.179999) (end 129 90.25) (width 0.3) (layer F.Cu) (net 12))
 (segment (start 130.18 81.4) (end 128.929999 82.650001) (width 0.3) (layer F.Cu) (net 12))
 (segment (start 128.929999 82.650001) (end 128.929999 90.179999) (width 0.3) (layer F.Cu) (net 12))
 (segment (start 156.287002 90.25) (end 157.826 88.711002) (width 0.3) (layer B.Cu) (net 12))
 (segment (start 157.826 88.711002) (end 157.826 84) (width 0.3) (layer B.Cu) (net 12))
 (segment (start 129 90.25) (end 156.287002 90.25) (width 0.3) (layer B.Cu) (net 12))
 (segment (start 139.749999 86.349999) (end 141 87.6) (width 0.3) (layer B.Cu) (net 14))
 (segment (start 135.129999 86.349999) (end 139.749999 86.349999) (width 0.3) (layer B.Cu) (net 14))
 (segment (start 132.72 83.94) (end 135.129999 86.349999) (width 0.3) (layer B.Cu) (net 14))
 (segment (start 132.72 81.4) (end 133.970001 82.650001) (width 0.3) (layer B.Cu) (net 2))
 (via (at 146.69 82.65) (size 0.8) (drill 0.4) (layers F.Cu B.Cu) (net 2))
 (segment (start 146.689999 82.650001) (end 146.69 82.65) (width 0.3) (layer B.Cu) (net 2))
 (segment (start 133.970001 82.650001) (end 146.689999 82.650001) (width 0.3) (layer B.Cu) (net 2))
 (segment (start 146.670001 88.350001) (end 150.2 91.88) (width 0.3) (layer F.Cu) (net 2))
 (segment (start 146.670001 82.669999) (end 146.670001 88.350001) (width 0.3) (layer F.Cu) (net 2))
 (segment (start 146.69 82.65) (end 146.670001 82.669999) (width 0.3) (layer F.Cu) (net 2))
 (segment (start 141.739989 85.799989) (end 143.54 87.6) (width 0.3) (layer B.Cu) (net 13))
 (segment (start 137.119989 85.799989) (end 141.739989 85.799989) (width 0.3) (layer B.Cu) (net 13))
 (segment (start 135.26 83.94) (end 137.119989 85.799989) (width 0.3) (layer B.Cu) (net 13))
 (segment (start 131.430001 83.379997) (end 131.430001 84.569999) (width 0.3) (layer F.Cu) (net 4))
 (segment (start 132.159997 82.650001) (end 131.430001 83.379997) (width 0.3) (layer F.Cu) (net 4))
 (segment (start 135.26 81.4) (end 134.009999 82.650001) (width 0.3) (layer F.Cu) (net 4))
 (segment (start 134.009999 82.650001) (end 132.159997 82.650001) (width 0.3) (layer F.Cu) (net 4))
 (via (at 130.5 98.75) (size 0.8) (drill 0.4) (layers F.Cu B.Cu) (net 4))
 (segment (start 131.430001 84.569999) (end 130.5 85.5) (width 0.3) (layer F.Cu) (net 4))
 (segment (start 130.5 85.5) (end 130.5 98.75) (width 0.3) (layer F.Cu) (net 4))
 (segment (start 145.15 98.75) (end 145.2 98.8) (width 0.3) (layer B.Cu) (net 4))
 (segment (start 130.5 98.75) (end 145.15 98.75) (width 0.3) (layer B.Cu) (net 4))
 (segment (start 148.13 101.73) (end 145.2 98.8) (width 0.3) (layer B.Cu) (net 4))
 (segment (start 148.63 101.73) (end 148.13 101.73) (width 0.3) (layer B.Cu) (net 4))
 (via (at 152 88.050001) (size 0.8) (drill 0.4) (layers F.Cu B.Cu) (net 16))
 (segment (start 146.961999 85.190001) (end 149.821999 88.050001) (width 0.3) (layer B.Cu) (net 16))
 (segment (start 137.8 83.94) (end 139.050001 85.190001) (width 0.3) (layer B.Cu) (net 16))
 (segment (start 149.821999 88.050001) (end 152 88.050001) (width 0.3) (layer B.Cu) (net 16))
 (segment (start 139.050001 85.190001) (end 146.961999 85.190001) (width 0.3) (layer B.Cu) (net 16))
 (segment (start 152 98.56) (end 156.29 102.85) (width 0.3) (layer F.Cu) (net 16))
 (segment (start 152 88.050001) (end 152 98.56) (width 0.3) (layer F.Cu) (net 16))
 (segment (start 132 89.099998) (end 132 94) (width 0.3) (layer F.Cu) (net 15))
 (via (at 132 94) (size 0.8) (drill 0.4) (layers F.Cu B.Cu) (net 15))
 (segment (start 140.34 83.94) (end 138.719252 85.560748) (width 0.3) (layer F.Cu) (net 15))
 (segment (start 135.53925 85.560748) (end 132 89.099998) (width 0.3) (layer F.Cu) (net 15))
 (segment (start 138.719252 85.560748) (end 135.53925 85.560748) (width 0.3) (layer F.Cu) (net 15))
 (segment (start 122.71 97.433998) (end 122.71 98.34) (width 0.3) (layer B.Cu) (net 15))
 (segment (start 124.503999 95.639999) (end 122.71 97.433998) (width 0.3) (layer B.Cu) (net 15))
 (segment (start 125.816003 95.639999) (end 124.503999 95.639999) (width 0.3) (layer B.Cu) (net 15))
 (segment (start 127.456002 94) (end 125.816003 95.639999) (width 0.3) (layer B.Cu) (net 15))
 (segment (start 132 94) (end 127.456002 94) (width 0.3) (layer B.Cu) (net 15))
 (segment (start 145.2 84.16) (end 145.42 83.94) (width 0.25) (layer F.Cu) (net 7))
 (segment (start 145.42 91.38) (end 145.2 91.6) (width 0.3) (layer F.Cu) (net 7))
 (segment (start 145.42 83.94) (end 145.42 91.38) (width 0.3) (layer F.Cu) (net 7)))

